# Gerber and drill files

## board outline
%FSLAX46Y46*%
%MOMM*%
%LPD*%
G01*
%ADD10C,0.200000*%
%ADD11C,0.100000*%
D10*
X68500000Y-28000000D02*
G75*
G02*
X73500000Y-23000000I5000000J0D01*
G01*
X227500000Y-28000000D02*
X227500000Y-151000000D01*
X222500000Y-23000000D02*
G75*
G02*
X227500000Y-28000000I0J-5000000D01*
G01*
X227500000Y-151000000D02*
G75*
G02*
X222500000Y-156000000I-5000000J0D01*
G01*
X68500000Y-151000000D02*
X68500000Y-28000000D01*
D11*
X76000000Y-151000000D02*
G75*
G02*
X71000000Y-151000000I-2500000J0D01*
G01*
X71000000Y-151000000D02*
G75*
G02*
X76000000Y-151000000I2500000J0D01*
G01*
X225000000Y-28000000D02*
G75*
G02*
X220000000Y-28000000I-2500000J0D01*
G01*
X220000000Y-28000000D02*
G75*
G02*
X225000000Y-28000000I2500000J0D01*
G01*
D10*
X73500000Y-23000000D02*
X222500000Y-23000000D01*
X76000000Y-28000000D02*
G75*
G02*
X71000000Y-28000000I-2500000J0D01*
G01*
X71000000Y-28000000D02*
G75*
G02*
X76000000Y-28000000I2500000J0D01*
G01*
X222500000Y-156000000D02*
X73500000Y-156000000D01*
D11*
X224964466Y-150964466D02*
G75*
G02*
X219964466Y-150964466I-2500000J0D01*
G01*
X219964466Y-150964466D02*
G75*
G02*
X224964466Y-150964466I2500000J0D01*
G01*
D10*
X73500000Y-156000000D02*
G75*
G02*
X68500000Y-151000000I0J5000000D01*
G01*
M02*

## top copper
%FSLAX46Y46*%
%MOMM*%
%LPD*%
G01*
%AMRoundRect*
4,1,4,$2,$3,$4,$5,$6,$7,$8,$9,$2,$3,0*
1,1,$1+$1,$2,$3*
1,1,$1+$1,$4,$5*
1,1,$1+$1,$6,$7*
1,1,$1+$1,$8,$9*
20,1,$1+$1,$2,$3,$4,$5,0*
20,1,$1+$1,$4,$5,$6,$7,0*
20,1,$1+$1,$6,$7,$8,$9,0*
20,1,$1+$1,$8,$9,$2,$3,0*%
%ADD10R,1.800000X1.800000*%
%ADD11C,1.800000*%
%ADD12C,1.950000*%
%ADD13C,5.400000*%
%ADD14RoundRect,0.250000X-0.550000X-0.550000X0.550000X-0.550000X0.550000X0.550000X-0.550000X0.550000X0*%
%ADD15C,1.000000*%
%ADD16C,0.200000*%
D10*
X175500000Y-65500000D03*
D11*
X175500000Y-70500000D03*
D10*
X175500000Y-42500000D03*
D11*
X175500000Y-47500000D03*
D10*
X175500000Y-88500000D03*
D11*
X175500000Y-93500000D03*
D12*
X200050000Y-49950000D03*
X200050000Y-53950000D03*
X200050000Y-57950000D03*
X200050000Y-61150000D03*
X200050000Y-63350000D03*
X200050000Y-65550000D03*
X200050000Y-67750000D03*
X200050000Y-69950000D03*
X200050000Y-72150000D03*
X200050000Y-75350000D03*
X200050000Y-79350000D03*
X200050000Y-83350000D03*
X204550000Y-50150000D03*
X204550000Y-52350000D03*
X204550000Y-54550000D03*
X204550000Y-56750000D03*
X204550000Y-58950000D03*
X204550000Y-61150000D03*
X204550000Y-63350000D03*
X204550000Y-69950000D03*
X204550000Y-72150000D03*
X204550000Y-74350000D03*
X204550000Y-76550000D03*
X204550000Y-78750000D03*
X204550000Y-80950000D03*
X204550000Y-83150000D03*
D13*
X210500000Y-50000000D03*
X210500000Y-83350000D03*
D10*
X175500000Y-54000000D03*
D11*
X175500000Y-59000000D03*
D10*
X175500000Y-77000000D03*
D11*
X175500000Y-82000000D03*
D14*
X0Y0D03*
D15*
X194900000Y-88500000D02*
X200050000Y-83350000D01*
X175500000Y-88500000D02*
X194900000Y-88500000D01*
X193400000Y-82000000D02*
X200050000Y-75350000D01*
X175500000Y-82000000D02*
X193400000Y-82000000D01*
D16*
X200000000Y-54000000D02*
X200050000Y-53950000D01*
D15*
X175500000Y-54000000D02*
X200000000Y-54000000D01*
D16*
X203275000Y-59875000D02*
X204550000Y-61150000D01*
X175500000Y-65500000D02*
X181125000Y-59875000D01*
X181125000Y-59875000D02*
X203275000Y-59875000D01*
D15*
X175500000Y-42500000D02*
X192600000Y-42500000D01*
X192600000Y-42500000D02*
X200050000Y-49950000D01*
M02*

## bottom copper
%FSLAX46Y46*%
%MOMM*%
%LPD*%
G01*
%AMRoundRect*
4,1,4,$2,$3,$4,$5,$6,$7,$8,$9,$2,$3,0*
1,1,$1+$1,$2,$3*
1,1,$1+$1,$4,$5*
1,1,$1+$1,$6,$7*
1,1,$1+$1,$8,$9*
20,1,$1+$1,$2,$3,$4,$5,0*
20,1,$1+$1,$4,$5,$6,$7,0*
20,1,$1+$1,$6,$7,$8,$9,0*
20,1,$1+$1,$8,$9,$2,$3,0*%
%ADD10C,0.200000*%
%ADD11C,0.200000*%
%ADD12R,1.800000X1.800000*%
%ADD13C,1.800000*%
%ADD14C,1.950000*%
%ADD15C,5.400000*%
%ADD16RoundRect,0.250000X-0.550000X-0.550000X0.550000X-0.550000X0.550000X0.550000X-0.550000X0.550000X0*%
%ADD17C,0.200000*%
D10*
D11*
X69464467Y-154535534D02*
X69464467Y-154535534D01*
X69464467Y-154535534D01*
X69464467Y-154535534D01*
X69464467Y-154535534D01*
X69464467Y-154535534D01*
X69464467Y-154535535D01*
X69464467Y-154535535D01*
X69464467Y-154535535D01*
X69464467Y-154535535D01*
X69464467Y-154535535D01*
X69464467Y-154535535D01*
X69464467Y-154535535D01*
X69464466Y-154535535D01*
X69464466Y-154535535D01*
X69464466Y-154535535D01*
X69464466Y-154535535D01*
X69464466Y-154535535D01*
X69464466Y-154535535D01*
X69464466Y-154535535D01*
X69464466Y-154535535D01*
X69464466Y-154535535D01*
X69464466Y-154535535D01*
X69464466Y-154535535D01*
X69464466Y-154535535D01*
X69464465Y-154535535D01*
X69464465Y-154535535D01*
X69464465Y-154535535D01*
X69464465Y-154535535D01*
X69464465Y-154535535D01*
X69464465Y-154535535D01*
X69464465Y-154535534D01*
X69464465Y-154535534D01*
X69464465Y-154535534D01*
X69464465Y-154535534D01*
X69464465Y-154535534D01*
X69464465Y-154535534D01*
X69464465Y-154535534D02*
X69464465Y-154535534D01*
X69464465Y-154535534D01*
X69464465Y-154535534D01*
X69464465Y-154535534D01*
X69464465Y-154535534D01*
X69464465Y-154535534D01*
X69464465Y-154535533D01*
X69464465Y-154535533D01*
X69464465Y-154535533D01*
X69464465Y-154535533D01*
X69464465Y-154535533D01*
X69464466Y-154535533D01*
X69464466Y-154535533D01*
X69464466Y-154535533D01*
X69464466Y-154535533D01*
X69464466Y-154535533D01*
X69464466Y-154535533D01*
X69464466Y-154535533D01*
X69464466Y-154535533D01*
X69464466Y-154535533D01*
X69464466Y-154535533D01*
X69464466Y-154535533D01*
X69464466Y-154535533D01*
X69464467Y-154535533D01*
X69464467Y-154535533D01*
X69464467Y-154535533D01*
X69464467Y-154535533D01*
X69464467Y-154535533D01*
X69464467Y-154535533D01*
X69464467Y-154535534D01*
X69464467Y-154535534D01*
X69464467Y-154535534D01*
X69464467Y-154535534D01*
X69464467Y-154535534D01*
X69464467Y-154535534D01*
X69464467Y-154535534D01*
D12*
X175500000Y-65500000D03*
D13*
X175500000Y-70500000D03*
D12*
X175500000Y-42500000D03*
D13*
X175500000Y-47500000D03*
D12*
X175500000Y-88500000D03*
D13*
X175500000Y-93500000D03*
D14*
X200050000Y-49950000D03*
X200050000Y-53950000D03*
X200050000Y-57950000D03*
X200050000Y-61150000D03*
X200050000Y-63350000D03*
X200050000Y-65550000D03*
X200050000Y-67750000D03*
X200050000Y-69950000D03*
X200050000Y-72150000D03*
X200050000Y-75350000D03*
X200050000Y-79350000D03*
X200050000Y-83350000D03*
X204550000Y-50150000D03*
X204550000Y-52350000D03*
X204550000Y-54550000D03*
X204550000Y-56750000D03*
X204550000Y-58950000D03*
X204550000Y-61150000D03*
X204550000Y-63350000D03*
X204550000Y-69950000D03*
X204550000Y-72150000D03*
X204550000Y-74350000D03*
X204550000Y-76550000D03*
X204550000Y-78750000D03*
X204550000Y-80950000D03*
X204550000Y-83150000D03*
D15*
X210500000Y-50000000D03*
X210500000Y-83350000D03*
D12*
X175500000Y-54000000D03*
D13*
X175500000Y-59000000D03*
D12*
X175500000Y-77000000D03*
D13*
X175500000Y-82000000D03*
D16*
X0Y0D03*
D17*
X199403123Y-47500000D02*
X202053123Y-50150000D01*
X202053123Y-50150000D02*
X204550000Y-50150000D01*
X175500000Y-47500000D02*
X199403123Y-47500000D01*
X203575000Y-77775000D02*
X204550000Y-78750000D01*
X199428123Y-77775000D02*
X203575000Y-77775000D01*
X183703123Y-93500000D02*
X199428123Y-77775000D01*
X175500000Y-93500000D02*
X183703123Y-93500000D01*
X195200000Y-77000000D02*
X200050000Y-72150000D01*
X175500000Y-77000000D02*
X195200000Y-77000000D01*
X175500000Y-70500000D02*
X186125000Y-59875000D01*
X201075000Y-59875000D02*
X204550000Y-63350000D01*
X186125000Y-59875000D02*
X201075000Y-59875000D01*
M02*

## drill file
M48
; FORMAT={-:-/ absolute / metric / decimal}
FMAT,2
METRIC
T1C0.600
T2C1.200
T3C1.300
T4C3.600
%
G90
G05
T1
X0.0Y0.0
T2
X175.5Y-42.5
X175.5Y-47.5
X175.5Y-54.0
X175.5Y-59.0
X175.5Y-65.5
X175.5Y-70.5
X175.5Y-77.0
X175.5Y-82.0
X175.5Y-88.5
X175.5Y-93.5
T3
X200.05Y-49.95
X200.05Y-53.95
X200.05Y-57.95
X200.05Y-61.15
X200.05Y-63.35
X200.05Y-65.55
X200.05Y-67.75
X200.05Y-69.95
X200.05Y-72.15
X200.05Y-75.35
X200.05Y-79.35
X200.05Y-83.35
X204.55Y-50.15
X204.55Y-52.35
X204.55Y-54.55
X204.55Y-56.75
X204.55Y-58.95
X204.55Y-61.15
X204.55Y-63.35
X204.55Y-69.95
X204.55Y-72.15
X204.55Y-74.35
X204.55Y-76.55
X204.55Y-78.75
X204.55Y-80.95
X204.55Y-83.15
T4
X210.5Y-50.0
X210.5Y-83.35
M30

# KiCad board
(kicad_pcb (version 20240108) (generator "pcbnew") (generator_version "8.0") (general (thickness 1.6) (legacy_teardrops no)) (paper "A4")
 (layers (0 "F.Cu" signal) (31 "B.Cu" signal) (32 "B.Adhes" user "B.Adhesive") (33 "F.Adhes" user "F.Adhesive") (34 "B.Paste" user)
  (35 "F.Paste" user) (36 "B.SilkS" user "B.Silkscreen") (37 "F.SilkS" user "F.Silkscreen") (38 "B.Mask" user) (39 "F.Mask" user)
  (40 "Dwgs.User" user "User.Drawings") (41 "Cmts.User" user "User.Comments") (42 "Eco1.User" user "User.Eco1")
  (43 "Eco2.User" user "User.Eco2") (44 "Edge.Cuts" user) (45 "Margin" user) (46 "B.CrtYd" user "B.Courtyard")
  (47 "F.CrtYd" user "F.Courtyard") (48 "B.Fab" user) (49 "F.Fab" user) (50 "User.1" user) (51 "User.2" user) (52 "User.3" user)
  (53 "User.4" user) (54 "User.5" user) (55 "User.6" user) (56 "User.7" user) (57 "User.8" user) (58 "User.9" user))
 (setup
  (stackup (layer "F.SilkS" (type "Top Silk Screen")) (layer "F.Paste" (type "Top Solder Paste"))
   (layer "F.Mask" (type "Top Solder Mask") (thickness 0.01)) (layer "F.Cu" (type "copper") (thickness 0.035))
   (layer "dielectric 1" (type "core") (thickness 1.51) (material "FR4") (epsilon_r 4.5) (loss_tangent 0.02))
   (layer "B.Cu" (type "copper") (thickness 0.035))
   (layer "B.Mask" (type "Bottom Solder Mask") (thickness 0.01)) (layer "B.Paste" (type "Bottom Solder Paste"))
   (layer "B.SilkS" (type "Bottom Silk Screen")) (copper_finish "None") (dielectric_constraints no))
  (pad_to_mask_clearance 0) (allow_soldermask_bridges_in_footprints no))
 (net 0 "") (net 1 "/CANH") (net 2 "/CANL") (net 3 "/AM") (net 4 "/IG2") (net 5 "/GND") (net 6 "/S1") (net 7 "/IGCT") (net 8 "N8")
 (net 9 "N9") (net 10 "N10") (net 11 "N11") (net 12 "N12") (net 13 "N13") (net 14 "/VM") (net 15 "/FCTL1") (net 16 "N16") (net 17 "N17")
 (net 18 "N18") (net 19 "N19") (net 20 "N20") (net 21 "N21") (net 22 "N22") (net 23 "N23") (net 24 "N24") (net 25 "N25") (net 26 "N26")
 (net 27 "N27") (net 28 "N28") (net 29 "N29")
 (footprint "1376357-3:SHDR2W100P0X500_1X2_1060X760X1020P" (layer "F.Cu") (at 175.5 65.5 -90)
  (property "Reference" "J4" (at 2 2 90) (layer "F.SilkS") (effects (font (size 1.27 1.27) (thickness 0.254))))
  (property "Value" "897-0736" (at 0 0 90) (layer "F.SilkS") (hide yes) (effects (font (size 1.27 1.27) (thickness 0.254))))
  (pad "1" thru_hole rect (at 0 0 270) (size 1.8 1.8) (drill 1.2) (layers "*.Cu" "*.Mask") (remove_unused_layers no) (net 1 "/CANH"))
  (pad "2" thru_hole circle (at 5 0 270) (size 1.8 1.8) (drill 1.2) (layers "*.Cu" "*.Mask") (remove_unused_layers no) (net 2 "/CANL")))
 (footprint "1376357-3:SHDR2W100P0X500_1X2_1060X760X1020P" (layer "F.Cu") (at 175.5 42.5 -90)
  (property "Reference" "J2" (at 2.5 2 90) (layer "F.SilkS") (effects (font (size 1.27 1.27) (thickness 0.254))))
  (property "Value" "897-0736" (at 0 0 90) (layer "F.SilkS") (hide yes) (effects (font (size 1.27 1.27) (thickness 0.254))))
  (pad "1" thru_hole rect (at 0 0 270) (size 1.8 1.8) (drill 1.2) (layers "*.Cu" "*.Mask") (remove_unused_layers no) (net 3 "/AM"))
  (pad "2" thru_hole circle (at 5 0 270) (size 1.8 1.8) (drill 1.2) (layers "*.Cu" "*.Mask") (remove_unused_layers no) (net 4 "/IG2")))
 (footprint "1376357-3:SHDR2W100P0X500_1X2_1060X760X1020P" (layer "F.Cu") (at 175.5 88.5 -90)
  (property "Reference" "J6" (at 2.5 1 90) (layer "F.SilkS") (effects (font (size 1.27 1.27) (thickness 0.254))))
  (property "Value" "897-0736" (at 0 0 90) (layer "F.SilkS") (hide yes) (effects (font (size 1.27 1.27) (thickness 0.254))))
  (pad "1" thru_hole rect (at 0 0 270) (size 1.8 1.8) (drill 1.2) (layers "*.Cu" "*.Mask") (remove_unused_layers no) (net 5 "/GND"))
  (pad "2" thru_hole circle (at 5 0 270) (size 1.8 1.8) (drill 1.2) (layers "*.Cu" "*.Mask") (remove_unused_layers no) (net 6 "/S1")))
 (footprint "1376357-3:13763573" (layer "F.Cu") (at 200.05 50)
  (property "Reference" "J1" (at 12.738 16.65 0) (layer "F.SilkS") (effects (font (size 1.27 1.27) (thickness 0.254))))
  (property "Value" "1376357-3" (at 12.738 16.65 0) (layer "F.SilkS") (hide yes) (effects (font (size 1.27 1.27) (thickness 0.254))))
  (pad "1" thru_hole circle (at 0 -0.05) (size 1.95 1.95) (drill 1.3) (layers "*.Cu" "*.Mask") (remove_unused_layers no) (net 3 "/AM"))
  (pad "2" thru_hole circle (at 0 3.95) (size 1.95 1.95) (drill 1.3) (layers "*.Cu" "*.Mask") (remove_unused_layers no) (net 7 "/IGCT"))
  (pad "3" thru_hole circle (at 0 7.95) (size 1.95 1.95) (drill 1.3) (layers "*.Cu" "*.Mask") (remove_unused_layers no) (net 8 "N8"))
  (pad "4" thru_hole circle (at 0 11.15) (size 1.95 1.95) (drill 1.3) (layers "*.Cu" "*.Mask") (remove_unused_layers no) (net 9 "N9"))
  (pad "5" thru_hole circle (at 0 13.35) (size 1.95 1.95) (drill 1.3) (layers "*.Cu" "*.Mask") (remove_unused_layers no) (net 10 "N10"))
  (pad "6" thru_hole circle (at 0 15.55) (size 1.95 1.95) (drill 1.3) (layers "*.Cu" "*.Mask") (remove_unused_layers no) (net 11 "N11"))
  (pad "7" thru_hole circle (at 0 17.75) (size 1.95 1.95) (drill 1.3) (layers "*.Cu" "*.Mask") (remove_unused_layers no) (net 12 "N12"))
  (pad "8" thru_hole circle (at 0 19.95) (size 1.95 1.95) (drill 1.3) (layers "*.Cu" "*.Mask") (remove_unused_layers no) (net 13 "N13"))
  (pad "9" thru_hole circle (at 0 22.15) (size 1.95 1.95) (drill 1.3) (layers "*.Cu" "*.Mask") (remove_unused_layers no) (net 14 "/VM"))
  (pad "10" thru_hole circle (at 0 25.35) (size 1.95 1.95) (drill 1.3) (layers "*.Cu" "*.Mask") (remove_unused_layers no) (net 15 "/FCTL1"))
  (pad "11" thru_hole circle (at 0 29.35) (size 1.95 1.95) (drill 1.3) (layers "*.Cu" "*.Mask") (remove_unused_layers no) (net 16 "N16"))
  (pad "12" thru_hole circle (at 0 33.35) (size 1.95 1.95) (drill 1.3) (layers "*.Cu" "*.Mask") (remove_unused_layers no) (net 5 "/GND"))
  (pad "13" thru_hole circle (at 4.5 0.15) (size 1.95 1.95) (drill 1.3) (layers "*.Cu" "*.Mask") (remove_unused_layers no) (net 4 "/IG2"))
  (pad "14" thru_hole circle (at 4.5 2.35) (size 1.95 1.95) (drill 1.3) (layers "*.Cu" "*.Mask") (remove_unused_layers no) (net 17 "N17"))
  (pad "15" thru_hole circle (at 4.5 4.55) (size 1.95 1.95) (drill 1.3) (layers "*.Cu" "*.Mask") (remove_unused_layers no) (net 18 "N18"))
  (pad "16" thru_hole circle (at 4.5 6.75) (size 1.95 1.95) (drill 1.3) (layers "*.Cu" "*.Mask") (remove_unused_layers no) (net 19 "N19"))
  (pad "17" thru_hole circle (at 4.5 8.95) (size 1.95 1.95) (drill 1.3) (layers "*.Cu" "*.Mask") (remove_unused_layers no) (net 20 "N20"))
  (pad "18" thru_hole circle (at 4.5 11.15) (size 1.95 1.95) (drill 1.3) (layers "*.Cu" "*.Mask") (remove_unused_layers no) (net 1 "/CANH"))
  (pad "19" thru_hole circle (at 4.5 13.35) (size 1.95 1.95) (drill 1.3) (layers "*.Cu" "*.Mask") (remove_unused_layers no) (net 2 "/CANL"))
  (pad "20" thru_hole circle (at 4.5 19.95) (size 1.95 1.95) (drill 1.3) (layers "*.Cu" "*.Mask") (remove_unused_layers no) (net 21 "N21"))
  (pad "21" thru_hole circle (at 4.5 22.15) (size 1.95 1.95) (drill 1.3) (layers "*.Cu" "*.Mask") (remove_unused_layers no) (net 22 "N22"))
  (pad "22" thru_hole circle (at 4.5 24.35) (size 1.95 1.95) (drill 1.3) (layers "*.Cu" "*.Mask") (remove_unused_layers no) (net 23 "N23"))
  (pad "23" thru_hole circle (at 4.5 26.55) (size 1.95 1.95) (drill 1.3) (layers "*.Cu" "*.Mask") (remove_unused_layers no) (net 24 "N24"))
  (pad "24" thru_hole circle (at 4.5 28.75) (size 1.95 1.95) (drill 1.3) (layers "*.Cu" "*.Mask") (remove_unused_layers no) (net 6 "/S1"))
  (pad "25" thru_hole circle (at 4.5 30.95) (size 1.95 1.95) (drill 1.3) (layers "*.Cu" "*.Mask") (remove_unused_layers no) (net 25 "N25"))
  (pad "26" thru_hole circle (at 4.5 33.15) (size 1.95 1.95) (drill 1.3) (layers "*.Cu" "*.Mask") (remove_unused_layers no) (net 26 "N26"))
  (pad "MH1" thru_hole circle (at 10.45 0) (size 5.4 5.4) (drill 3.6) (layers "*.Cu" "*.Mask") (remove_unused_layers no) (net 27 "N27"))
  (pad "MH2" thru_hole circle (at 10.45 33.35) (size 5.4 5.4) (drill 3.6) (layers "*.Cu" "*.Mask") (remove_unused_layers no) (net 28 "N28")))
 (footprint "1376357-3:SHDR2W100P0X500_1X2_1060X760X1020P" (layer "F.Cu") (at 175.5 54 -90)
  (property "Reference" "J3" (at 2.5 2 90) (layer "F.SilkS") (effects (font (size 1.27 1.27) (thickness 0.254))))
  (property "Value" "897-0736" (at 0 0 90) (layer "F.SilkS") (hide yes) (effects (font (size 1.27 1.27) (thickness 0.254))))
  (pad "1" thru_hole rect (at 0 0 270) (size 1.8 1.8) (drill 1.2) (layers "*.Cu" "*.Mask") (remove_unused_layers no) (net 7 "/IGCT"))
  (pad "2" thru_hole circle (at 5 0 270) (size 1.8 1.8) (drill 1.2) (layers "*.Cu" "*.Mask") (remove_unused_layers no) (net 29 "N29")))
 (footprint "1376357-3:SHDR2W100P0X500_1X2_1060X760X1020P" (layer "F.Cu") (at 175.5 77 -90)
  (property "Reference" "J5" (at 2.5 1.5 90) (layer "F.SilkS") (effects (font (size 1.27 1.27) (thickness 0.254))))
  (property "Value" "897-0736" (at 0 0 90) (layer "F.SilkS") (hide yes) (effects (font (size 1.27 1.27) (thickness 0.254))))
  (pad "1" thru_hole rect (at 0 0 270) (size 1.8 1.8) (drill 1.2) (layers "*.Cu" "*.Mask") (remove_unused_layers no) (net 14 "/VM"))
  (pad "2" thru_hole circle (at 5 0 270) (size 1.8 1.8) (drill 1.2) (layers "*.Cu" "*.Mask") (remove_unused_layers no) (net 15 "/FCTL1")))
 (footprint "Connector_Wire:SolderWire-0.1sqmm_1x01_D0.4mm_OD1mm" (layer "F.Cu") (at 0 0)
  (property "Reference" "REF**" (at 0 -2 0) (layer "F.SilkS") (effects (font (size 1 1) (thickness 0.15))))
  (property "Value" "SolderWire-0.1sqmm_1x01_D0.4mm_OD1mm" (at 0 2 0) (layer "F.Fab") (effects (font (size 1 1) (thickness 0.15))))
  (pad "1" thru_hole roundrect (at 0 0) (size 1.6 1.6) (drill 0.6) (layers "*.Cu" "*.Mask") (remove_unused_layers no)
   (roundrect_rratio 0.15625)))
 (gr_arc (start 69.464466 154.535534) (mid 69.464466 154.535534) (end 69.464466 154.535534) (stroke (width 0.2) (type default))
  (layer "B.Cu"))
 (gr_arc (start 68.5 28) (mid 69.964466 24.464466) (end 73.5 23) (stroke (width 0.2) (type default)) (layer "Edge.Cuts"))
 (gr_line (start 227.5 28) (end 227.5 151) (stroke (width 0.2) (type default)) (layer "Edge.Cuts"))
 (gr_arc (start 222.5 23) (mid 226.035534 24.464466) (end 227.5 28) (stroke (width 0.2) (type default)) (layer "Edge.Cuts"))
 (gr_arc (start 227.5 151) (mid 226.035534 154.535534) (end 222.5 156) (stroke (width 0.2) (type default)) (layer "Edge.Cuts"))
 (gr_line (start 68.5 151) (end 68.5 28) (stroke (width 0.2) (type default)) (layer "Edge.Cuts"))
 (gr_circle (center 73.5 151) (end 76 151) (stroke (width 0.1) (type default)) (fill none) (layer "Edge.Cuts"))
 (gr_circle (center 222.5 28) (end 225 28) (stroke (width 0.1) (type default)) (fill none) (layer "Edge.Cuts"))
 (gr_line (start 73.5 23) (end 222.5 23) (stroke (width 0.2) (type default)) (layer "Edge.Cuts"))
 (gr_circle (center 73.5 28) (end 76 28) (stroke (width 0.2) (type default)) (fill none) (layer "Edge.Cuts"))
 (gr_line (start 222.5 156) (end 73.5 156) (stroke (width 0.2) (type default)) (layer "Edge.Cuts"))
 (gr_circle (center 222.464466 150.964466) (end 224.964466 150.964466) (stroke (width 0.1) (type default)) (fill none) (layer "Edge.Cuts"))
 (gr_arc (start 73.5 156) (mid 69.964466 154.535534) (end 68.5 151) (stroke (width 0.2) (type default)) (layer "Edge.Cuts"))
 (segment (start 199.403123 47.5) (end 202.053123 50.15) (width 0.2) (layer "B.Cu") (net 4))
 (segment (start 202.053123 50.15) (end 204.55 50.15) (width 0.2) (layer "B.Cu") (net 4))
 (segment (start 175.5 47.5) (end 199.403123 47.5) (width 0.2) (layer "B.Cu") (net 4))
 (segment (start 194.9 88.5) (end 200.05 83.35) (width 1) (layer "F.Cu") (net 5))
 (segment (start 175.5 88.5) (end 194.9 88.5) (width 1) (layer "F.Cu") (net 5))
 (segment (start 203.575 77.775) (end 204.55 78.75) (width 0.2) (layer "B.Cu") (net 6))
 (segment (start 199.428123 77.775) (end 203.575 77.775) (width 0.2) (layer "B.Cu") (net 6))
 (segment (start 183.703123 93.5) (end 199.428123 77.775) (width 0.2) (layer "B.Cu") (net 6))
 (segment (start 175.5 93.5) (end 183.703123 93.5) (width 0.2) (layer "B.Cu") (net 6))
 (segment (start 193.4 82) (end 200.05 75.35) (width 1) (layer "F.Cu") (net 15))
 (segment (start 175.5 82) (end 193.4 82) (width 1) (layer "F.Cu") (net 15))
 (segment (start 200 54) (end 200.05 53.95) (width 0.2) (layer "F.Cu") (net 7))
 (segment (start 175.5 54) (end 200 54) (width 1) (layer "F.Cu") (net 7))
 (segment (start 195.2 77) (end 200.05 72.15) (width 0.2) (layer "B.Cu") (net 14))
 (segment (start 175.5 77) (end 195.2 77) (width 0.2) (layer "B.Cu") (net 14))
 (segment (start 175.5 70.5) (end 186.125 59.875) (width 0.2) (layer "B.Cu") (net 2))
 (segment (start 201.075 59.875) (end 204.55 63.35) (width 0.2) (layer "B.Cu") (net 2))
 (segment (start 186.125 59.875) (end 201.075 59.875) (width 0.2) (layer "B.Cu") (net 2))
 (segment (start 203.275 59.875) (end 204.55 61.15) (width 0.2) (layer "F.Cu") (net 1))
 (segment (start 175.5 65.5) (end 181.125 59.875) (width 0.2) (layer "F.Cu") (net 1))
 (segment (start 181.125 59.875) (end 203.275 59.875) (width 0.2) (layer "F.Cu") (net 1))
 (segment (start 175.5 42.5) (end 192.6 42.5) (width 1) (layer "F.Cu") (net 3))
 (segment (start 192.6 42.5) (end 200.05 49.95) (width 1) (layer "F.Cu") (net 3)))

